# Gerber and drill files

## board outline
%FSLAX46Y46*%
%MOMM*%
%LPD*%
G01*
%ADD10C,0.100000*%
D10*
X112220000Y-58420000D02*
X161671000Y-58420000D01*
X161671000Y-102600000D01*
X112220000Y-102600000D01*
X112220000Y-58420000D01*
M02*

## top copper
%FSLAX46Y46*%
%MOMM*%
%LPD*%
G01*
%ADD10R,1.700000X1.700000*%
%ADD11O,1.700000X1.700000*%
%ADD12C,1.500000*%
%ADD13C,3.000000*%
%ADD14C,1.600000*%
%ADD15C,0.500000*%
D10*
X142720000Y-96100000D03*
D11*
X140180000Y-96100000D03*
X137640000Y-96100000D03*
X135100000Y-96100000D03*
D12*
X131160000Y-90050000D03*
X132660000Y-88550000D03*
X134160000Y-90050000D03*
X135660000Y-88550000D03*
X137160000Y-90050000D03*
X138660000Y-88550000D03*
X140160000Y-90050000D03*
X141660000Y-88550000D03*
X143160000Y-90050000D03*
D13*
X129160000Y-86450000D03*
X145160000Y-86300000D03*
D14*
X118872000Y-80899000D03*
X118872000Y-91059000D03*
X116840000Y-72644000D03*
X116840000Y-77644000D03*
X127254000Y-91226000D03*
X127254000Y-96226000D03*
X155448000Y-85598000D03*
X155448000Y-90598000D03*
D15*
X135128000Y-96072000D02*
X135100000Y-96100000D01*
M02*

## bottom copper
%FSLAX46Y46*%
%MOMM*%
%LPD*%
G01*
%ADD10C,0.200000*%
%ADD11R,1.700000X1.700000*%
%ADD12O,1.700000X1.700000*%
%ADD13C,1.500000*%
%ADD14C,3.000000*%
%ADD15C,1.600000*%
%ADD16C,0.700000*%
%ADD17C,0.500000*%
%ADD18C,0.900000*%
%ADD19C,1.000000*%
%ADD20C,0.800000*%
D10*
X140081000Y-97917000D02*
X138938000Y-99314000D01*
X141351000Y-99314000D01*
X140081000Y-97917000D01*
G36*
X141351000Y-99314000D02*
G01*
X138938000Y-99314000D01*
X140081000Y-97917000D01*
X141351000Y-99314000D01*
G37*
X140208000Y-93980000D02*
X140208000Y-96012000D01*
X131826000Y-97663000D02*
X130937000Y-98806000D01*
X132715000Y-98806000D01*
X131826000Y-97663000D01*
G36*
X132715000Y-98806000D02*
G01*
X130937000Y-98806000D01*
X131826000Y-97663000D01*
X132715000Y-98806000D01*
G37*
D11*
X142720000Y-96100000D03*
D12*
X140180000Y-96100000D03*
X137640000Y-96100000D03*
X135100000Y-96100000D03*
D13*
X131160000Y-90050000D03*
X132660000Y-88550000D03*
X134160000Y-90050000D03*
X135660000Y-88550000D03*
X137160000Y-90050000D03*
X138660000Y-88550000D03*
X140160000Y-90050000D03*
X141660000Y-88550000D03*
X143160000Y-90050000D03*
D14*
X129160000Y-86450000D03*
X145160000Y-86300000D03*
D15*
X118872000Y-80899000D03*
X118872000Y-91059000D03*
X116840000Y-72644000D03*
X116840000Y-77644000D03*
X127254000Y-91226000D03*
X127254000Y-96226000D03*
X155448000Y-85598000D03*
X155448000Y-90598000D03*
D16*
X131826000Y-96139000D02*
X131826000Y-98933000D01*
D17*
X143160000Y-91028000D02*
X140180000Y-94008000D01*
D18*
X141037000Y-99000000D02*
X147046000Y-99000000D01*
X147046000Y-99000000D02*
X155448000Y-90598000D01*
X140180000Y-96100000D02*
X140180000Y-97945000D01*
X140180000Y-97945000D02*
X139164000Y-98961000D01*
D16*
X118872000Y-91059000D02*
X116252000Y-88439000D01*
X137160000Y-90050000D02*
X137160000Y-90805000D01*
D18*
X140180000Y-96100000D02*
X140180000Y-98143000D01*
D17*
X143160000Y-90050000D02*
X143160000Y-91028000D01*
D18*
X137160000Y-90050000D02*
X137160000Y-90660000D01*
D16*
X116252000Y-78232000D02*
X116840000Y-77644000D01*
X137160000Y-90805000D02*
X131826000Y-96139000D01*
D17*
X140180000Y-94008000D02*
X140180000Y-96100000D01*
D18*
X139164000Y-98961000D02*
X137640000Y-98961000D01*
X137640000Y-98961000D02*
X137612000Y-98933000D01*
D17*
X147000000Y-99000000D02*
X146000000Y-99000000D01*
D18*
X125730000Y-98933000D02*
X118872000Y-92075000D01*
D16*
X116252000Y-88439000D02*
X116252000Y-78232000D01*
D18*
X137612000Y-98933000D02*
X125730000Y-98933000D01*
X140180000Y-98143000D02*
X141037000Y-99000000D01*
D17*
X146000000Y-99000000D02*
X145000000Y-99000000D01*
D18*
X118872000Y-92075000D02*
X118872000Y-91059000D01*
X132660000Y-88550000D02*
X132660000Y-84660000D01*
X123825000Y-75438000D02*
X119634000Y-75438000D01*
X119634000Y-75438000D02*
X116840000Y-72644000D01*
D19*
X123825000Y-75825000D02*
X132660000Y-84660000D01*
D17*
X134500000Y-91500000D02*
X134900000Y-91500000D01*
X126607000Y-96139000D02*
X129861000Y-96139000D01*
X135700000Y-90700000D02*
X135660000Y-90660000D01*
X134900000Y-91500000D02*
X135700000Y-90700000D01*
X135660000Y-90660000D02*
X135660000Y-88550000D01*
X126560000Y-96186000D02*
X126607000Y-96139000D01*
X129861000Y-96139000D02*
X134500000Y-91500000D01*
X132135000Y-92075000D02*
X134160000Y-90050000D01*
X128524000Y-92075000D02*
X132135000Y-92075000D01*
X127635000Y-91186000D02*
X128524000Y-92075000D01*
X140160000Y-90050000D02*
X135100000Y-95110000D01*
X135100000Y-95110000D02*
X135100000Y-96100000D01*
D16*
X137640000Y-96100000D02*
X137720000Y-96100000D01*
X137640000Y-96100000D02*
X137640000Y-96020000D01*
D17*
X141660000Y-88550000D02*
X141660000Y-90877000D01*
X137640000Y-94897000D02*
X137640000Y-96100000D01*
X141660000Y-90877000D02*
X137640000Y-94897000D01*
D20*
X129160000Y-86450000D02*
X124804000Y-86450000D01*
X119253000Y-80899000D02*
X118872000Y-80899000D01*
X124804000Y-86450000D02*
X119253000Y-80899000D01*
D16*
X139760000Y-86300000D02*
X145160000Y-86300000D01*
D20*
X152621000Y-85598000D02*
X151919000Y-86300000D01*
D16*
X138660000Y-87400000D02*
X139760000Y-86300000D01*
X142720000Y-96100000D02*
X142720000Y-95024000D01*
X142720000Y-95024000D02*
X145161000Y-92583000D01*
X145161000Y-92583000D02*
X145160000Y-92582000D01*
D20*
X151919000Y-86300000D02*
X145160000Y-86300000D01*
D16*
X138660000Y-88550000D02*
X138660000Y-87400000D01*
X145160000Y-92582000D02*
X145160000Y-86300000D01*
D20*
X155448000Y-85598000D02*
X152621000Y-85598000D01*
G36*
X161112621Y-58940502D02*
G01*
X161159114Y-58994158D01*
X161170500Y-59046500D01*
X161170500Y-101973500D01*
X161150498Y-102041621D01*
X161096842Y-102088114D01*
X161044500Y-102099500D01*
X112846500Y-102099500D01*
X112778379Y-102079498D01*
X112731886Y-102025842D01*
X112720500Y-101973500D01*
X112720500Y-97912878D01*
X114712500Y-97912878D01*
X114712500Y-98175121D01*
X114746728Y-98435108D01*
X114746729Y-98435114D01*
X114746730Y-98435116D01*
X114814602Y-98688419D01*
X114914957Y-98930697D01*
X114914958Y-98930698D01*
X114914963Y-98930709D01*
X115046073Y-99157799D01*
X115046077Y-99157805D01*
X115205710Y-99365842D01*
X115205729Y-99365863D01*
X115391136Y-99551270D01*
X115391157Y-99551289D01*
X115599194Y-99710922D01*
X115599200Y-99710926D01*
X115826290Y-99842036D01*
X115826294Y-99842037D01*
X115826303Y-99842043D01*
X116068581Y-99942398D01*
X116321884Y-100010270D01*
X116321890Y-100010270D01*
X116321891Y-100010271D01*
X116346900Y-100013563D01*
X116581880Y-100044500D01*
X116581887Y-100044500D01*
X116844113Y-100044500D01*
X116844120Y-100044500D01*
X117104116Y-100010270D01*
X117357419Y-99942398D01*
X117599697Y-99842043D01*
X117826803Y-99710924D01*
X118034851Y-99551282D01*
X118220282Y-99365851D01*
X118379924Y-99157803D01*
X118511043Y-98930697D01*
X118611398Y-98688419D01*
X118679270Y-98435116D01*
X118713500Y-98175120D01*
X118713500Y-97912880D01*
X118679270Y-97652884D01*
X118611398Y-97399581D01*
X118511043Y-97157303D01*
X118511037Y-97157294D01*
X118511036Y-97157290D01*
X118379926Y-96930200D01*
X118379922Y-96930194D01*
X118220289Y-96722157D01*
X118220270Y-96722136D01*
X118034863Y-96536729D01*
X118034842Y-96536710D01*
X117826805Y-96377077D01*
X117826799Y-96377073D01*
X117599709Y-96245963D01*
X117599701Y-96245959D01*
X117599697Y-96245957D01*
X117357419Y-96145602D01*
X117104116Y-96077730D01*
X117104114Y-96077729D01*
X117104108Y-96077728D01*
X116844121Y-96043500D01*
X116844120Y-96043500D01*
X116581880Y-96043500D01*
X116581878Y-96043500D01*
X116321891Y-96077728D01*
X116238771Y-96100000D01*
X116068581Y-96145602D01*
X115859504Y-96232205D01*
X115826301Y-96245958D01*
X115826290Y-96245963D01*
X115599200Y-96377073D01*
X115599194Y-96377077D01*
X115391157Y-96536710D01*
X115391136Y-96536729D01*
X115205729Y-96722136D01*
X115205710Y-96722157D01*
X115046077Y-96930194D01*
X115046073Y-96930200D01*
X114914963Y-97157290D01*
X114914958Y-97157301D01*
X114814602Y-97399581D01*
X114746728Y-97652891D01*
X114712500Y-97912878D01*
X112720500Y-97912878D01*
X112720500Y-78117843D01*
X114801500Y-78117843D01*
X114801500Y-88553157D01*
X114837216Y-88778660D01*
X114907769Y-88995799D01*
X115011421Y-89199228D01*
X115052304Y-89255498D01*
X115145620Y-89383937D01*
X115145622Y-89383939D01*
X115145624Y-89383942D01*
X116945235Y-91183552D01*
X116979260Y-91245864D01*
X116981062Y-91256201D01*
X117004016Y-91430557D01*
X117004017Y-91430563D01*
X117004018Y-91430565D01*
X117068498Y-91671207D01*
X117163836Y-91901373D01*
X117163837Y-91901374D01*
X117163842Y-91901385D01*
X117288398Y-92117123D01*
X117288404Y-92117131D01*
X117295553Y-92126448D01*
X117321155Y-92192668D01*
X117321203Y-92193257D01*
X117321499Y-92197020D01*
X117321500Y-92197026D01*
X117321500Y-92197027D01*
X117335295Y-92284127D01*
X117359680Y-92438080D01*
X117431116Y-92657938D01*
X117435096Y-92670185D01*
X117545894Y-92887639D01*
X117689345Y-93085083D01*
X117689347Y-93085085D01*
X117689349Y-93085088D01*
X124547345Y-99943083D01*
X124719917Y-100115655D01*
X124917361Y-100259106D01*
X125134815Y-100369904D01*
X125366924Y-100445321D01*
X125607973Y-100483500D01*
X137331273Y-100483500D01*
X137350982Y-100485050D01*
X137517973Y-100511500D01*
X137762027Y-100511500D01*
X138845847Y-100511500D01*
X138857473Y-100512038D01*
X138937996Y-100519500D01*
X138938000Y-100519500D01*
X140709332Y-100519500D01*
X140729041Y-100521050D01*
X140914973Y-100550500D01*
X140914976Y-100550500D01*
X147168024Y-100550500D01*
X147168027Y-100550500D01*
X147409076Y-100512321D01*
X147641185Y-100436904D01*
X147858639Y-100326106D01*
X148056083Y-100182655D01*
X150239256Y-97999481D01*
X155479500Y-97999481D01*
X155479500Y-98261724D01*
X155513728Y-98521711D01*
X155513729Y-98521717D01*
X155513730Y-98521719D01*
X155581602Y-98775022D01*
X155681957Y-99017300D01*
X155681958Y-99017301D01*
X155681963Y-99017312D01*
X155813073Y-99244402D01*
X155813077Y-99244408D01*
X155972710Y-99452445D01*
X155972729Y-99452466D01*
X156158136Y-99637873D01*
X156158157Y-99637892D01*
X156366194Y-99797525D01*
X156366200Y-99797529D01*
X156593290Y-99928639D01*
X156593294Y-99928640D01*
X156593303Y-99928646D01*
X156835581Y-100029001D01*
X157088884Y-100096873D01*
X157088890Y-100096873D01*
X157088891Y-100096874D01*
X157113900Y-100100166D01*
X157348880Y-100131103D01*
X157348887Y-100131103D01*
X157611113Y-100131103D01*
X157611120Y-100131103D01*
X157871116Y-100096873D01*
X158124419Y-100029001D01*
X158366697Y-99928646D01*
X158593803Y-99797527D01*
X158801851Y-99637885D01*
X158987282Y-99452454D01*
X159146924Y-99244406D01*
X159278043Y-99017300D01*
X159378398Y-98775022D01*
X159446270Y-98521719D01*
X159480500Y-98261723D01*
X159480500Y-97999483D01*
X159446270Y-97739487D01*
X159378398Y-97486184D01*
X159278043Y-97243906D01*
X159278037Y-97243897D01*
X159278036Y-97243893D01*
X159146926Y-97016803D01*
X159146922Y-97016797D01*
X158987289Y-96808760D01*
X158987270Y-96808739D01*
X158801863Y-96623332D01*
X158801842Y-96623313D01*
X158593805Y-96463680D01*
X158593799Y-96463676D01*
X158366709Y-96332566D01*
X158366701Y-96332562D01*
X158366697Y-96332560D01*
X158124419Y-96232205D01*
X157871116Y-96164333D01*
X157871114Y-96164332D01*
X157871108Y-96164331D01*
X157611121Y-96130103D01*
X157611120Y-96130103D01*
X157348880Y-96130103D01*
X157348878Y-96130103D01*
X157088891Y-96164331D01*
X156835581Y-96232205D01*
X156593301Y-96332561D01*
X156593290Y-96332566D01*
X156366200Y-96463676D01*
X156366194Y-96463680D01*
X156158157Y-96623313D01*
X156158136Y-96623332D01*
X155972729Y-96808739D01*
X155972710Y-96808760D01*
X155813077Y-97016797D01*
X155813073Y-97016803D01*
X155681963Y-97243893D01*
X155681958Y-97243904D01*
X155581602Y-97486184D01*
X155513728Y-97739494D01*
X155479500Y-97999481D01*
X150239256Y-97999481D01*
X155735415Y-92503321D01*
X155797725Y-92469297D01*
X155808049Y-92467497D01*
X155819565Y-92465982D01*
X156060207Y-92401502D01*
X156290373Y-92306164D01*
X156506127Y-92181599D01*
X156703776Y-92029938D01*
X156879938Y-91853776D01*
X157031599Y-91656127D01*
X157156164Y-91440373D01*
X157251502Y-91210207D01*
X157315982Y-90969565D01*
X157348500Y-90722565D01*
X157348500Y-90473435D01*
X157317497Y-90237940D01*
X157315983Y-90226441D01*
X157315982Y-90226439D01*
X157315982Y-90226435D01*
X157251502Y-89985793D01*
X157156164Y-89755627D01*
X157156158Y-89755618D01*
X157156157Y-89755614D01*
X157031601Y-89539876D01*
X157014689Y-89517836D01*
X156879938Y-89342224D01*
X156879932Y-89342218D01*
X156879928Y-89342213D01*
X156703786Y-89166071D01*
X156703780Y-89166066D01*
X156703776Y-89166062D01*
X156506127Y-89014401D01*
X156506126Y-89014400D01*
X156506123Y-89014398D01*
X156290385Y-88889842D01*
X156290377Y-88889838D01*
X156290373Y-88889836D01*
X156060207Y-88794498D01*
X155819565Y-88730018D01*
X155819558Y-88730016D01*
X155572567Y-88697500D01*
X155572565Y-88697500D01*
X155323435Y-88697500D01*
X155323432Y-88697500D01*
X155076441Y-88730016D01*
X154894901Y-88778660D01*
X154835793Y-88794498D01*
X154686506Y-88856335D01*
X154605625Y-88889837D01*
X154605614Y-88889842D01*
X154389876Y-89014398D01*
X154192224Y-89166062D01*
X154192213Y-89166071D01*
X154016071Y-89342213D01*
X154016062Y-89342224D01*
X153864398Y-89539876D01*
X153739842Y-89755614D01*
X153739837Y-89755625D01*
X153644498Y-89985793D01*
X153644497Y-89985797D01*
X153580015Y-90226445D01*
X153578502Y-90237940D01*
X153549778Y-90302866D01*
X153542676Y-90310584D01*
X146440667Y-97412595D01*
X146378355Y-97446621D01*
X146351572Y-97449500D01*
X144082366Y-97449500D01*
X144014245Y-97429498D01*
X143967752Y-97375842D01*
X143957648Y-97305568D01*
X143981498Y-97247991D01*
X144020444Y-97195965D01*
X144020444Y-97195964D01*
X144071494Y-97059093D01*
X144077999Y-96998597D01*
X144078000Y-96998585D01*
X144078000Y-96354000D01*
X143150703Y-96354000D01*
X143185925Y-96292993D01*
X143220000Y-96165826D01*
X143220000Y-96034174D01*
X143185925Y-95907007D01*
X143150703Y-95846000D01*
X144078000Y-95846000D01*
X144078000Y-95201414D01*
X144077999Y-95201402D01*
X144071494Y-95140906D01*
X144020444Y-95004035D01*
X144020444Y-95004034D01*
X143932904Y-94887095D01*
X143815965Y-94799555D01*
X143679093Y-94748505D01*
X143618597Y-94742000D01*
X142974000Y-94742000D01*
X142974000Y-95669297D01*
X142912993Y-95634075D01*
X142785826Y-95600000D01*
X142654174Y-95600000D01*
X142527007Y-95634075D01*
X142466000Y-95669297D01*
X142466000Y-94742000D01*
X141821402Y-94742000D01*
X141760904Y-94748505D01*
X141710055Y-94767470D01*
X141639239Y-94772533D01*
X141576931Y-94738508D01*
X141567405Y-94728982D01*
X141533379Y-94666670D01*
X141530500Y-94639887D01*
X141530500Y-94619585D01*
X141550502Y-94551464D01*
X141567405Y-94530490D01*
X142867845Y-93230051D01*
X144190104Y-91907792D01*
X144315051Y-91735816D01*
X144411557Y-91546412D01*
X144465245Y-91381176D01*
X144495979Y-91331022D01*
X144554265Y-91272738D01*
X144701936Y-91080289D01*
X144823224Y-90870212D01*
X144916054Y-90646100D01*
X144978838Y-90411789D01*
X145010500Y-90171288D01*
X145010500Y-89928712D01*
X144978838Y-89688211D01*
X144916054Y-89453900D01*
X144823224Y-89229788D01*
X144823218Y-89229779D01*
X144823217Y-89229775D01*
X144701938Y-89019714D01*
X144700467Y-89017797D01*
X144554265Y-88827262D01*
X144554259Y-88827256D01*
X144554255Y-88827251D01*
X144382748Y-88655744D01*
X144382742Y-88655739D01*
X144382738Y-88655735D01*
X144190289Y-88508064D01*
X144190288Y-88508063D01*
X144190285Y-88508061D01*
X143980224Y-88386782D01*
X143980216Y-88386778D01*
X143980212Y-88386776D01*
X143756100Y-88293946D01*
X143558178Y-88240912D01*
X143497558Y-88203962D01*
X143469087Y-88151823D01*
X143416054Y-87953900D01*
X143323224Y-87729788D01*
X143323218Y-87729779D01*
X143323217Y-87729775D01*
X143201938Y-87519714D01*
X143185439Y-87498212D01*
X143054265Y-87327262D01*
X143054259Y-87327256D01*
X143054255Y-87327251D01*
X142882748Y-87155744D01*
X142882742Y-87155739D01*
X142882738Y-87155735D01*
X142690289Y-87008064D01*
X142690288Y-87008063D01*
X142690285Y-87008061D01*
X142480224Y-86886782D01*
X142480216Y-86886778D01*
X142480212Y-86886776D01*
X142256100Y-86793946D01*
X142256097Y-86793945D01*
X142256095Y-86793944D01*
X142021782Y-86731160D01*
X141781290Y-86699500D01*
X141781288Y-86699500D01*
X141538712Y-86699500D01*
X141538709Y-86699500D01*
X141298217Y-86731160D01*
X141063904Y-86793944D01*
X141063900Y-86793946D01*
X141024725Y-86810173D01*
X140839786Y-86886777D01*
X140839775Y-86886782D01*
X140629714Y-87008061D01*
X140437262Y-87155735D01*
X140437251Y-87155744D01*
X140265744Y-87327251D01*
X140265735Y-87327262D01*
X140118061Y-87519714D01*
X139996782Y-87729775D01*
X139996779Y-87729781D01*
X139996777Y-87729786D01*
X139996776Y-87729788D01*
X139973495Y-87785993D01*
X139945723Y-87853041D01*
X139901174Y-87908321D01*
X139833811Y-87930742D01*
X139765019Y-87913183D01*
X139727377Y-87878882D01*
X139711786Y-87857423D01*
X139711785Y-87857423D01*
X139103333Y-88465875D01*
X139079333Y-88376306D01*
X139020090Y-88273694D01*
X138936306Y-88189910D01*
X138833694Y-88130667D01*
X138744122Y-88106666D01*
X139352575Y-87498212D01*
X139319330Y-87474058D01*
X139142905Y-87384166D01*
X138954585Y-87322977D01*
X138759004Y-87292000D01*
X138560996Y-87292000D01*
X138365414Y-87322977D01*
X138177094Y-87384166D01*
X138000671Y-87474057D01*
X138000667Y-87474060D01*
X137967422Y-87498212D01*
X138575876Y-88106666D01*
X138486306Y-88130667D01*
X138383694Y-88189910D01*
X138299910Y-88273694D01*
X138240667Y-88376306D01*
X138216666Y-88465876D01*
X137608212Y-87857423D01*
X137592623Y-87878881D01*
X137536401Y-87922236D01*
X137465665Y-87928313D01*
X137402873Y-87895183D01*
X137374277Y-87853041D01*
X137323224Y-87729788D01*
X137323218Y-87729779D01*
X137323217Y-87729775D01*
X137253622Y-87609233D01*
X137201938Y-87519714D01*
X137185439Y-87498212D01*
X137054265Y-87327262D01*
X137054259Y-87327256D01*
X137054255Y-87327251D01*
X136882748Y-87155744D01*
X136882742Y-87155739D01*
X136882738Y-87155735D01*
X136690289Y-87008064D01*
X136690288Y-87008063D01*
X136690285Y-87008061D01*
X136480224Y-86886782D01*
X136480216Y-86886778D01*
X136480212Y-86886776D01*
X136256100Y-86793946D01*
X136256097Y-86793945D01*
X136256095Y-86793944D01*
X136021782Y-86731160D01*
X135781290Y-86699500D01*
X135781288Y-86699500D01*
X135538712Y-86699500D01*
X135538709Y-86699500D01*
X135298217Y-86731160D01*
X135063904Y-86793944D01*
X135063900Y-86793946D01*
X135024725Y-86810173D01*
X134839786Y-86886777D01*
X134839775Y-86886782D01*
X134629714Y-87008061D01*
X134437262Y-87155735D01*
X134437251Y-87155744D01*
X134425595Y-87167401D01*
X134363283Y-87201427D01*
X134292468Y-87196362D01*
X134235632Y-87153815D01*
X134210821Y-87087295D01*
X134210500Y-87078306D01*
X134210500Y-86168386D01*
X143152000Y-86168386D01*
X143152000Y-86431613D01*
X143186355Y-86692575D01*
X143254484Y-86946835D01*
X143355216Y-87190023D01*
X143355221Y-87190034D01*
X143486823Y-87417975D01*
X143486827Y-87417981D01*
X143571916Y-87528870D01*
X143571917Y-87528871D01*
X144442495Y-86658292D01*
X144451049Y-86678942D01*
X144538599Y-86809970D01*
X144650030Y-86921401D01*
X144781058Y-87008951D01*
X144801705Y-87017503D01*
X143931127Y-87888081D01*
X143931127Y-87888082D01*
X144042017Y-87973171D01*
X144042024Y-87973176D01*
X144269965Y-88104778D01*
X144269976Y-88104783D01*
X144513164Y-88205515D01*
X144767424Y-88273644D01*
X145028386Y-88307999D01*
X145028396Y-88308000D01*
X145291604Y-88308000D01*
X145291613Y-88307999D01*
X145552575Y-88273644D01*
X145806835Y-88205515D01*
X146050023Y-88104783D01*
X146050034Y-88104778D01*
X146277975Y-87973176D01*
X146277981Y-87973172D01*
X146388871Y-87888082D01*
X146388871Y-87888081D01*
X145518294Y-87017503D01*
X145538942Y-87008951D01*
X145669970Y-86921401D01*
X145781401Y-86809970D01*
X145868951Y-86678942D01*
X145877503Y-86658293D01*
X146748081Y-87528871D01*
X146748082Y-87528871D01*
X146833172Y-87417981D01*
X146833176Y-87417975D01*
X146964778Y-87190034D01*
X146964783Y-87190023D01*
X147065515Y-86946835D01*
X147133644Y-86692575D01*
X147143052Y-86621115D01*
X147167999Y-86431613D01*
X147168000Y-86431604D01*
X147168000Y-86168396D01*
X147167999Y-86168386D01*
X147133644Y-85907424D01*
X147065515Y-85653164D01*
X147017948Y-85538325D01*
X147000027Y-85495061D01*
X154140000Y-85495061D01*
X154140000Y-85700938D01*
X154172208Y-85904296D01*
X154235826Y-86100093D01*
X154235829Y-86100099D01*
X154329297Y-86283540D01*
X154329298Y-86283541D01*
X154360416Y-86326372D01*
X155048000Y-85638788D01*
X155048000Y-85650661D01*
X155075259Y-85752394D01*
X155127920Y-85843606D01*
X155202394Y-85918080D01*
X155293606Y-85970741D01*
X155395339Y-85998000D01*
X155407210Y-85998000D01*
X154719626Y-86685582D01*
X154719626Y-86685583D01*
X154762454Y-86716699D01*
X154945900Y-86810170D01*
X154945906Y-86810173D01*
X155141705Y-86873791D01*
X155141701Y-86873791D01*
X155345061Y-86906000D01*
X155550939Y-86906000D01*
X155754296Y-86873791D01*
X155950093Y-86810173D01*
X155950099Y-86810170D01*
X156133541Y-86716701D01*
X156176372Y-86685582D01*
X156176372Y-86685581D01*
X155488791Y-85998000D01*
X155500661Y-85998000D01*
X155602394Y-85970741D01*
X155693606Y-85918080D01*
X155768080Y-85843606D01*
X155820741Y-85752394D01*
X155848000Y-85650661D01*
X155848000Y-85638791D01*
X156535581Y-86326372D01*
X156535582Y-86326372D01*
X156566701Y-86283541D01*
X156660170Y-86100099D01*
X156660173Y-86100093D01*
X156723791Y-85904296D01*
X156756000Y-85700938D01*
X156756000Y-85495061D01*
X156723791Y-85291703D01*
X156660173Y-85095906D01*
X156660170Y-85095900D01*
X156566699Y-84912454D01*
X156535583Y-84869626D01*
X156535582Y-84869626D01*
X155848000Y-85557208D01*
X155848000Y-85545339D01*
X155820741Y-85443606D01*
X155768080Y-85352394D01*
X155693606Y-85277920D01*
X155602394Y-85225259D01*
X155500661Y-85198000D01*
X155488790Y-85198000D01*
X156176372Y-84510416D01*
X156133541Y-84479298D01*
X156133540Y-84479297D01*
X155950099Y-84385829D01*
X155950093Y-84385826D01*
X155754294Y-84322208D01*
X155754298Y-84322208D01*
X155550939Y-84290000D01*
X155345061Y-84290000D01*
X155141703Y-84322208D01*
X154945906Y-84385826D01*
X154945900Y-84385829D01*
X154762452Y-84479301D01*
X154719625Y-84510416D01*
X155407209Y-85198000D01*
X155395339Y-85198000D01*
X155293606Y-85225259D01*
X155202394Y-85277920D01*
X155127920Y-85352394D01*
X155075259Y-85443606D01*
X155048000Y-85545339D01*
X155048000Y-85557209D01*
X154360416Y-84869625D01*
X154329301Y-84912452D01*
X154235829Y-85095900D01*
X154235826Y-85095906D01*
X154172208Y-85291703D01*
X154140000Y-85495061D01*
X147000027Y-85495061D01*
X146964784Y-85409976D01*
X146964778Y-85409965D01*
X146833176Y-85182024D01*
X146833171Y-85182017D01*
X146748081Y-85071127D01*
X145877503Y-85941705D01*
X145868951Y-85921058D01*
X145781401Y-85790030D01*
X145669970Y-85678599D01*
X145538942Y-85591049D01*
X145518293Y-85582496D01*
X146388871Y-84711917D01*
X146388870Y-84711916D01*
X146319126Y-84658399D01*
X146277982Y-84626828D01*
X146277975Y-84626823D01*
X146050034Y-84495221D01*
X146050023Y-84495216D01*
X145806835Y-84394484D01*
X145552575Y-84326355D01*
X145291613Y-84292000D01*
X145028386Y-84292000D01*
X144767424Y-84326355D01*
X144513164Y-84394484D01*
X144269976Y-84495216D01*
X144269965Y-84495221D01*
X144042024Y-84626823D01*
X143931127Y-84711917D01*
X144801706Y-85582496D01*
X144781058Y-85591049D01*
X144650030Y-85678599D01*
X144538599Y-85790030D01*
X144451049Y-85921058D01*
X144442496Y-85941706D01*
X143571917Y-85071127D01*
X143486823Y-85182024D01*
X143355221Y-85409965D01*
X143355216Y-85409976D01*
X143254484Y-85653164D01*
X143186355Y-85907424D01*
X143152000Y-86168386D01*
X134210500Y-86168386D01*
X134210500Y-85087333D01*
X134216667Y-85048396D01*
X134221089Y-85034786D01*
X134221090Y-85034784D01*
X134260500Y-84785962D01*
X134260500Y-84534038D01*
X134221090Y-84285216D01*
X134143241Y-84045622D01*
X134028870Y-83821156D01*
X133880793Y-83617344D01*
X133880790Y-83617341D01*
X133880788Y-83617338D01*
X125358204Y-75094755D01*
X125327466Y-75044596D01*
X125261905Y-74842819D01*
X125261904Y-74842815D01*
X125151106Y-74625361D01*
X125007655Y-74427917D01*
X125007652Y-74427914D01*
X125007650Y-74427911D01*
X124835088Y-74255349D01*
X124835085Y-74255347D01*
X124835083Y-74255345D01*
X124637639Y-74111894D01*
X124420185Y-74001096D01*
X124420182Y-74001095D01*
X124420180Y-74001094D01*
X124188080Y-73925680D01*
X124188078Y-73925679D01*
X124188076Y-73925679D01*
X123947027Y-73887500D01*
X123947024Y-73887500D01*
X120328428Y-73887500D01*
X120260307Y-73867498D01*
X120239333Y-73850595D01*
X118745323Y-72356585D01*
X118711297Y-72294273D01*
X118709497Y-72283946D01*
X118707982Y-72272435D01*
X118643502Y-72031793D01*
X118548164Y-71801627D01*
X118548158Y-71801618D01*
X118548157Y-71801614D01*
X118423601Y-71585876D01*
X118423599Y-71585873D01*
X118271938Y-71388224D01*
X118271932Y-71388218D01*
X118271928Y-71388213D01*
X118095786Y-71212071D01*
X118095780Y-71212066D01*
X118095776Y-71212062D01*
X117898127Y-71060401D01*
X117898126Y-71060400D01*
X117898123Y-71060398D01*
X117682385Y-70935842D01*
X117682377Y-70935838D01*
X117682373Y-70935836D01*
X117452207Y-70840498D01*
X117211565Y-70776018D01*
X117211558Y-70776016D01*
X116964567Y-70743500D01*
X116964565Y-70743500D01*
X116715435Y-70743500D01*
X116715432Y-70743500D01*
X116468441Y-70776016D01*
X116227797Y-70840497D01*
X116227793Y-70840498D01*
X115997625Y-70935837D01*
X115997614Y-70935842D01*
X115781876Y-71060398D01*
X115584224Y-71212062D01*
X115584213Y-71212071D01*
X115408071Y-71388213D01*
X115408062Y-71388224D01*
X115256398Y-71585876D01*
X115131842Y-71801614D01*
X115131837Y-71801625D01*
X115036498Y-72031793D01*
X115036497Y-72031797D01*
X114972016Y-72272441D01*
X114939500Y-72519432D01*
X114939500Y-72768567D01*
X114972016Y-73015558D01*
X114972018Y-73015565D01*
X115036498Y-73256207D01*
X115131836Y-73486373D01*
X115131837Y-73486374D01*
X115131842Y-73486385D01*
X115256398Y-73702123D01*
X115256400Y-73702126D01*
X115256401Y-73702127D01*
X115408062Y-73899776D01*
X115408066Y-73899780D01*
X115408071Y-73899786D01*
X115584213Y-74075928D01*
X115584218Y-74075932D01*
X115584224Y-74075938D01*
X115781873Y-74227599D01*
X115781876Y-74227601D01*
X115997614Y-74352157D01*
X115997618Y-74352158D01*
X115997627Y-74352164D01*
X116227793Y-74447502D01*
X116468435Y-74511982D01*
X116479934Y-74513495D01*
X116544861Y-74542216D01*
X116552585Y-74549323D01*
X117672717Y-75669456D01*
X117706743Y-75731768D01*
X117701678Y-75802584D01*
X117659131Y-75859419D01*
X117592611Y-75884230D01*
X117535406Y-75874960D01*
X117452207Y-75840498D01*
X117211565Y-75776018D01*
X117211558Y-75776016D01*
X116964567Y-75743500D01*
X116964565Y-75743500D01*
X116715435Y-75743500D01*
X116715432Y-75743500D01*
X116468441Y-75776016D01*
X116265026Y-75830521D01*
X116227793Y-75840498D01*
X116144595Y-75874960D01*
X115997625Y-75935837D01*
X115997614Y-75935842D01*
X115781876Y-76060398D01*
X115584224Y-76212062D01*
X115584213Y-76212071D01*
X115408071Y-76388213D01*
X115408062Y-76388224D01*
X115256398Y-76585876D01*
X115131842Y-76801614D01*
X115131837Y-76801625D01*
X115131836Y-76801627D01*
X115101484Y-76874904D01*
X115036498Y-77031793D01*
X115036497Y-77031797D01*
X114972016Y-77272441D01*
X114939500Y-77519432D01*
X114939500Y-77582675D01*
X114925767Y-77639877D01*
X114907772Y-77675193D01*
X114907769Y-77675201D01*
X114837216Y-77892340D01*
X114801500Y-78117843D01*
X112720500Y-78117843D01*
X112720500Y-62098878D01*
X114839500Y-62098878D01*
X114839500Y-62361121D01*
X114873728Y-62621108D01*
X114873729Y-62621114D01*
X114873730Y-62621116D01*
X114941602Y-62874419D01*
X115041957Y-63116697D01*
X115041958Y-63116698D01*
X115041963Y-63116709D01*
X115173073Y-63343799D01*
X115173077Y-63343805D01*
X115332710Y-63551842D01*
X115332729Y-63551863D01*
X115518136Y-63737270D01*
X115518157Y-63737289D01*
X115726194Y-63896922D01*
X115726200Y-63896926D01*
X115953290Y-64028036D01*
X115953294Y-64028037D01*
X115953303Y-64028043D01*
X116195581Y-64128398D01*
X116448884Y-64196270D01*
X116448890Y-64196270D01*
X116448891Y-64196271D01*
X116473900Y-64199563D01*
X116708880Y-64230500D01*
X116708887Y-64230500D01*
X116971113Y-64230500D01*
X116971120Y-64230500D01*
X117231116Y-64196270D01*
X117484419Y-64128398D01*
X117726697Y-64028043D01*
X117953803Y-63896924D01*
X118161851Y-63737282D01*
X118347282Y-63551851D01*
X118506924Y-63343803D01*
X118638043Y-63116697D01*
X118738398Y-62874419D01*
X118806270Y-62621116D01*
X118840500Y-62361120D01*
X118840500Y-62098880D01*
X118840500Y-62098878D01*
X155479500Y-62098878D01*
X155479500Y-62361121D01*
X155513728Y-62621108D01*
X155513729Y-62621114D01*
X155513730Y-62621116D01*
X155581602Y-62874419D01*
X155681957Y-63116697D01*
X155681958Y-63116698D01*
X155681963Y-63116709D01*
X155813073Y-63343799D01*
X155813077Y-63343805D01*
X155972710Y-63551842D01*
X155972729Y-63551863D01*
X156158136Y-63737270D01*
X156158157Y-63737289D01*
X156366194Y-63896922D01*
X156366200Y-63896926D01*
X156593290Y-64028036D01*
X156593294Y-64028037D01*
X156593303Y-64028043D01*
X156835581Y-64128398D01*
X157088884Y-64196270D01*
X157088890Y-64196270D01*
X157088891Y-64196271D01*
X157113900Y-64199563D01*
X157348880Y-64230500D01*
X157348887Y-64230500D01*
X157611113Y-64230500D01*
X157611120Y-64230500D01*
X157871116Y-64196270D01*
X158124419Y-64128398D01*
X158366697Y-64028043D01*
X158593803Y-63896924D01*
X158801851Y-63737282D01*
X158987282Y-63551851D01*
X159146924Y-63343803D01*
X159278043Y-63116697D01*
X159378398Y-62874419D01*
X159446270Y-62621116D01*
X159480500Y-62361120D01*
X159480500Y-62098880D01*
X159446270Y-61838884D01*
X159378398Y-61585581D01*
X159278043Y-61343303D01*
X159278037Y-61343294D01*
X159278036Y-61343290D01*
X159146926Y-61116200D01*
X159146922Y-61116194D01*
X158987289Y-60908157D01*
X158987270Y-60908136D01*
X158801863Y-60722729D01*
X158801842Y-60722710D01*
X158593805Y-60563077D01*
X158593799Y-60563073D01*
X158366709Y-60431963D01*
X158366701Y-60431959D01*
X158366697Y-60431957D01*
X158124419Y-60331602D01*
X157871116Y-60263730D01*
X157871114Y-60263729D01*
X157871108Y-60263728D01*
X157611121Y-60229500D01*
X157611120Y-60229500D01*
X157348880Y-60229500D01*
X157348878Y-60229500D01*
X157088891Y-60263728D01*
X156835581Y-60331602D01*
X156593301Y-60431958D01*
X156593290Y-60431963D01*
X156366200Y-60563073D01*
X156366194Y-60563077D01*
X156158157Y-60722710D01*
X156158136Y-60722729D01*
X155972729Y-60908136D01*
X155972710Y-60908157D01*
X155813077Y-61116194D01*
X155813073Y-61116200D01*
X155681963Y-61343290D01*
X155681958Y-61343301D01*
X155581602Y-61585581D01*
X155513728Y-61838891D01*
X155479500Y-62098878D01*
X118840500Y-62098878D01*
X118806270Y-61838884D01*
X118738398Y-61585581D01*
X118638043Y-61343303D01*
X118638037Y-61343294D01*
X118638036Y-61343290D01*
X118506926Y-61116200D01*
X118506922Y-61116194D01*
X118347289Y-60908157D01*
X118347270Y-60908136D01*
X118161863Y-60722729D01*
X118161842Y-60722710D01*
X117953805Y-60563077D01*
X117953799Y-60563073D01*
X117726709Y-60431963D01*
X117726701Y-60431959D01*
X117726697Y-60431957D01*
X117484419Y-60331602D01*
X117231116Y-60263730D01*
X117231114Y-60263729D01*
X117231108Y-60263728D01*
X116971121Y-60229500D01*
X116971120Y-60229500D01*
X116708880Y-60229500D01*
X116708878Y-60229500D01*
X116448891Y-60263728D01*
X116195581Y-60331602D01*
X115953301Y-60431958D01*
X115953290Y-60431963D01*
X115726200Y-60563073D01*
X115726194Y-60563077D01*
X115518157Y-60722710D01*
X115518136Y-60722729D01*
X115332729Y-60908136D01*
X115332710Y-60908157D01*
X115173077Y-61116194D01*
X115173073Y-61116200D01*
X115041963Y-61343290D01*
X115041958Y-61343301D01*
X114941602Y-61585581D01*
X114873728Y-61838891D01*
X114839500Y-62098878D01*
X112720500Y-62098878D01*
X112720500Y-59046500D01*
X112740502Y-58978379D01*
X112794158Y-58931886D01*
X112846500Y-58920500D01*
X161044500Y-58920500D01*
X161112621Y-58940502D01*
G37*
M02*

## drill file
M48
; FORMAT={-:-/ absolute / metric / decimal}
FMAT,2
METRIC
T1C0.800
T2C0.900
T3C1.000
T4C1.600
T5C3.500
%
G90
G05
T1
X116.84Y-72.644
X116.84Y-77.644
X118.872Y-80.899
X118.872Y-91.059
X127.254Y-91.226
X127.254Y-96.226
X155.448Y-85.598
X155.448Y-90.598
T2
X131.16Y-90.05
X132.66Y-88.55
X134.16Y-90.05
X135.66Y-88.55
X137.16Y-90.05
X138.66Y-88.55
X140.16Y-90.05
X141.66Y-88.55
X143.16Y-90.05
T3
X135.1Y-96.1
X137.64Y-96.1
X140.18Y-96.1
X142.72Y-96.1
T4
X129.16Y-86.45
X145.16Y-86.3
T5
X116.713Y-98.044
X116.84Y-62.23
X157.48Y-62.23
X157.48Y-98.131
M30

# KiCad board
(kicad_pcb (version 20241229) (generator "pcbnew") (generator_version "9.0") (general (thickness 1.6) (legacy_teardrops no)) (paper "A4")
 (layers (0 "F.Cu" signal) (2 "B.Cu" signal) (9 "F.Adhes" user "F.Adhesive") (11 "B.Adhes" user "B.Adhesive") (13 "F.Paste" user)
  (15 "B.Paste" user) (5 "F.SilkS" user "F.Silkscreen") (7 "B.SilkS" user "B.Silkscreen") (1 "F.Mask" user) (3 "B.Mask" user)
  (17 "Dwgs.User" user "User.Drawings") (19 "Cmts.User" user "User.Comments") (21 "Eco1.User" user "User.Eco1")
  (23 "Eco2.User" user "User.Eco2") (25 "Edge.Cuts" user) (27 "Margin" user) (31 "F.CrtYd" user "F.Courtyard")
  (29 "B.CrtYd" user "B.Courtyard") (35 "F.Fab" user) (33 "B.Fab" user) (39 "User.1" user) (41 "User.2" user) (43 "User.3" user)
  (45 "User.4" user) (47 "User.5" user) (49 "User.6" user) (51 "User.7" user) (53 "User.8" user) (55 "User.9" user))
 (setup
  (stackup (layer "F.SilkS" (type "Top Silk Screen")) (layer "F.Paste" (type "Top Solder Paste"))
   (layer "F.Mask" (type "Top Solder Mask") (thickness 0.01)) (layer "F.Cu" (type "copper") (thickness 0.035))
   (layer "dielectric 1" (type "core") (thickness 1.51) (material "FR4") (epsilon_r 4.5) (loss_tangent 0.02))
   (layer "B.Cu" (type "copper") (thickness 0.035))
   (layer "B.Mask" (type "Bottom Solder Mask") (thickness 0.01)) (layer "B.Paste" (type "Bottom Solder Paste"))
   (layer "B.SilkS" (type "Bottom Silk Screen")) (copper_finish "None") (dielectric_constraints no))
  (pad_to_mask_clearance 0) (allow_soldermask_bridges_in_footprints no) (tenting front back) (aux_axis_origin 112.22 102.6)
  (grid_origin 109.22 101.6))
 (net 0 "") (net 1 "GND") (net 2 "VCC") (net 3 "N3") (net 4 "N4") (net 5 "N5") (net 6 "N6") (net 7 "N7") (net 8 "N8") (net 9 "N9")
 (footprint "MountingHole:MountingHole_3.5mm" (layer "F.Cu") (at 157.48 62.23)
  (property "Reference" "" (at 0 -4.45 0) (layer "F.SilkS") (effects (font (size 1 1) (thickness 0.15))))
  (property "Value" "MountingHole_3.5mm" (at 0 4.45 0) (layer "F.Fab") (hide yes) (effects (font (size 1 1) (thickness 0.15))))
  (pad "" np_thru_hole circle (at 0 0) (size 3.5 3.5) (drill 3.5) (layers "*.Cu" "*.Mask")))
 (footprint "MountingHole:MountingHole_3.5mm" (layer "F.Cu") (at 157.48 98.130603)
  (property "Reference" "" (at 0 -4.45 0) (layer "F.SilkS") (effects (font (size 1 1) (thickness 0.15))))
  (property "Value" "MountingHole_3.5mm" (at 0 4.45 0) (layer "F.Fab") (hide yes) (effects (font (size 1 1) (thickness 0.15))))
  (pad "" np_thru_hole circle (at 0 0) (size 3.5 3.5) (drill 3.5) (layers "*.Cu" "*.Mask")))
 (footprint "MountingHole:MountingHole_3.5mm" (layer "F.Cu") (at 116.84 62.23)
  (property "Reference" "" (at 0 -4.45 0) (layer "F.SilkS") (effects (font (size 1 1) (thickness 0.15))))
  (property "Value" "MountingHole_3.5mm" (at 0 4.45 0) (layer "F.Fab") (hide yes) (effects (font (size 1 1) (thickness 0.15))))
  (pad "" np_thru_hole circle (at 0 0) (size 3.5 3.5) (drill 3.5) (layers "*.Cu" "*.Mask")))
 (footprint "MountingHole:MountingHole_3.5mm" (layer "F.Cu") (at 116.713 98.044)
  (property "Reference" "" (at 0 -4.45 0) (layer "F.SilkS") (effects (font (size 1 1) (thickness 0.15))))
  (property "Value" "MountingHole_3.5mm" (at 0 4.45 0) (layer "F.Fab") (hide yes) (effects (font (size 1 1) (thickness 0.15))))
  (pad "" np_thru_hole circle (at 0 0) (size 3.5 3.5) (drill 3.5) (layers "*.Cu" "*.Mask")))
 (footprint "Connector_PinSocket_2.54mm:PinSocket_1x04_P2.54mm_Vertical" (layer "F.Cu") (at 142.72 96.1 -90)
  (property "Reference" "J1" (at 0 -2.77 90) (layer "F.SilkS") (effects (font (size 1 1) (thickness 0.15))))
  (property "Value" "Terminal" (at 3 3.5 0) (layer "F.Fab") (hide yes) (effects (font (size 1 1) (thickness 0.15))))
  (pad "1" thru_hole rect (at 0 0 270) (size 1.7 1.7) (drill 1) (layers "*.Cu" "*.Mask") (remove_unused_layers no) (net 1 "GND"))
  (pad "2" thru_hole oval (at 0 2.54 270) (size 1.7 1.7) (drill 1) (layers "*.Cu" "*.Mask") (remove_unused_layers no) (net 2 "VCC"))
  (pad "3" thru_hole oval (at 0 5.08 270) (size 1.7 1.7) (drill 1) (layers "*.Cu" "*.Mask") (remove_unused_layers no) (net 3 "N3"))
  (pad "4" thru_hole oval (at 0 7.62 270) (size 1.7 1.7) (drill 1) (layers "*.Cu" "*.Mask") (remove_unused_layers no) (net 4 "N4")))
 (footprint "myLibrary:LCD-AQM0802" (layer "F.Cu") (at 137.16 88.55)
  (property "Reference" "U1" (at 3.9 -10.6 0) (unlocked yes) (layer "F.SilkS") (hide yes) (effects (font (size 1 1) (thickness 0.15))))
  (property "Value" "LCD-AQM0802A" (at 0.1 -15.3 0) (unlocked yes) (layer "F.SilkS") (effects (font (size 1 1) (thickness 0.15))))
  (pad "1" thru_hole circle (at -6 1.5) (size 1.5 1.5) (drill 0.9) (layers "*.Cu" "*.Mask") (remove_unused_layers no) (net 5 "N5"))
  (pad "2" thru_hole circle (at -4.5 0) (size 1.5 1.5) (drill 0.9) (layers "*.Cu" "*.Mask") (remove_unused_layers no) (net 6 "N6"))
  (pad "3" thru_hole circle (at -3 1.5) (size 1.5 1.5) (drill 0.9) (layers "*.Cu" "*.Mask") (remove_unused_layers no) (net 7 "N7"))
  (pad "4" thru_hole circle (at -1.5 0) (size 1.5 1.5) (drill 0.9) (layers "*.Cu" "*.Mask") (remove_unused_layers no) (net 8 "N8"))
  (pad "5" thru_hole circle (at 0 1.5) (size 1.5 1.5) (drill 0.9) (layers "*.Cu" "*.Mask") (remove_unused_layers no) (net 2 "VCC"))
  (pad "6" thru_hole circle (at 1.5 0) (size 1.5 1.5) (drill 0.9) (layers "*.Cu" "*.Mask") (remove_unused_layers no) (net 1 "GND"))
  (pad "7" thru_hole circle (at 3 1.5) (size 1.5 1.5) (drill 0.9) (layers "*.Cu" "*.Mask") (remove_unused_layers no) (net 4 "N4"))
  (pad "8" thru_hole circle (at 4.5 0) (size 1.5 1.5) (drill 0.9) (layers "*.Cu" "*.Mask") (remove_unused_layers no) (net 3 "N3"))
  (pad "9" thru_hole circle (at 6 1.5) (size 1.5 1.5) (drill 0.9) (layers "*.Cu" "*.Mask") (remove_unused_layers yes) (keep_end_layers yes)
   (zone_layer_connections) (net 2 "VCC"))
  (pad "10" thru_hole circle (at -8 -2.1 90) (size 3 3) (drill 1.6) (layers "*.Cu" "*.Mask") (remove_unused_layers yes)
   (keep_end_layers yes) (zone_layer_connections) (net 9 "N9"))
  (pad "11" thru_hole circle (at 8 -2.25 90) (size 3 3) (drill 1.6) (layers "*.Cu" "*.Mask") (remove_unused_layers no) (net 1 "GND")))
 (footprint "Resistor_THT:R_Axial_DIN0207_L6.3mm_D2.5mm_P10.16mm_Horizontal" (layer "B.Cu") (at 118.872 80.899 -90)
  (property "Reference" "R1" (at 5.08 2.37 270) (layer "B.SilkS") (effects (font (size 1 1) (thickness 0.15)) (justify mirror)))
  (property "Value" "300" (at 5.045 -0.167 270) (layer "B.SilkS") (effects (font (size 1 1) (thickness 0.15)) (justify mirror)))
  (pad "1" thru_hole circle (at 0 0 270) (size 1.6 1.6) (drill 0.8) (layers "*.Cu" "*.Mask") (remove_unused_layers no) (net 9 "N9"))
  (pad "2" thru_hole circle (at 10.16 0 270) (size 1.6 1.6) (drill 0.8) (layers "*.Cu" "*.Mask") (remove_unused_layers no) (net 2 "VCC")))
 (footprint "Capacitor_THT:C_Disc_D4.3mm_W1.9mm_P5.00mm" (layer "B.Cu") (at 116.84 72.644 -90)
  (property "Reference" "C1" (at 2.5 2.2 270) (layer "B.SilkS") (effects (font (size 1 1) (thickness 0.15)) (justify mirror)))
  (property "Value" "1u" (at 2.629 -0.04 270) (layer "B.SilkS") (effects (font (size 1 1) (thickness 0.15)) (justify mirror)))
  (pad "1" thru_hole circle (at 0 0 270) (size 1.6 1.6) (drill 0.8) (layers "*.Cu" "*.Mask") (remove_unused_layers no) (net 6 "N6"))
  (pad "2" thru_hole circle (at 5 0 270) (size 1.6 1.6) (drill 0.8) (layers "*.Cu" "*.Mask") (remove_unused_layers no) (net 2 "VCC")))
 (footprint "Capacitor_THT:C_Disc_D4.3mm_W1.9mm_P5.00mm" (layer "B.Cu") (at 127.254 91.226 -90)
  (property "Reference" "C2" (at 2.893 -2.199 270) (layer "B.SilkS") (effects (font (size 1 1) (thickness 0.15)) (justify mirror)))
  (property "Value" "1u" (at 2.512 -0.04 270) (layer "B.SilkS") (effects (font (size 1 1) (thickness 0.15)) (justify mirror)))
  (pad "1" thru_hole circle (at 0 0 270) (size 1.6 1.6) (drill 0.8) (layers "*.Cu" "*.Mask") (remove_unused_layers no) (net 7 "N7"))
  (pad "2" thru_hole circle (at 5 0 270) (size 1.6 1.6) (drill 0.8) (layers "*.Cu" "*.Mask") (remove_unused_layers no) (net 8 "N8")))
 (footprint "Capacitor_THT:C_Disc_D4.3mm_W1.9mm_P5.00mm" (layer "B.Cu") (at 155.448 85.598 -90)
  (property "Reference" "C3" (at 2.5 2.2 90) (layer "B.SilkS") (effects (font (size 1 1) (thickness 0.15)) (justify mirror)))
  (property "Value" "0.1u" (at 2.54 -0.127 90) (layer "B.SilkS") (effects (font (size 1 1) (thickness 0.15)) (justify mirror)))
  (pad "1" thru_hole circle (at 0 0 270) (size 1.6 1.6) (drill 0.8) (layers "*.Cu" "*.Mask") (remove_unused_layers no) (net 1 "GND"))
  (pad "2" thru_hole circle (at 5 0 270) (size 1.6 1.6) (drill 0.8) (layers "*.Cu" "*.Mask") (remove_unused_layers no) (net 2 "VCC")))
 (gr_poly
  (pts (xy 140.081 97.917) (xy 138.938 99.314) (xy 141.351 99.314)) (stroke (width 0.2) (type solid)) (fill yes) (layer "B.Cu") (net 2))
 (gr_line (start 140.208 93.98) (end 140.208 96.012) (stroke (width 0.2) (type default)) (layer "B.Cu") (net 2))
 (gr_poly
  (pts (xy 131.826 97.663) (xy 130.937 98.806) (xy 132.715 98.806)) (stroke (width 0.2) (type solid)) (fill yes) (layer "B.Cu") (net 2))
 (gr_rect (start 112.22 58.42) (end 161.671 102.6) (stroke (width 0.1) (type solid)) (fill no) (layer "Edge.Cuts"))
 (segment (start 131.826 96.139) (end 131.826 98.933) (width 0.7) (layer "B.Cu") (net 2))
 (segment (start 143.16 91.028) (end 140.18 94.008) (width 0.5) (layer "B.Cu") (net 2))
 (segment (start 141.037 99) (end 147.046 99) (width 0.9) (layer "B.Cu") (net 2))
 (segment (start 147.046 99) (end 155.448 90.598) (width 0.9) (layer "B.Cu") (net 2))
 (segment (start 140.18 96.1) (end 140.18 97.945) (width 0.9) (layer "B.Cu") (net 2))
 (segment (start 140.18 97.945) (end 139.164 98.961) (width 0.9) (layer "B.Cu") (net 2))
 (segment (start 118.872 91.059) (end 116.252 88.439) (width 0.7) (layer "B.Cu") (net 2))
 (segment (start 137.16 90.05) (end 137.16 90.805) (width 0.7) (layer "B.Cu") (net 2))
 (segment (start 140.18 96.1) (end 140.18 98.143) (width 0.9) (layer "B.Cu") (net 2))
 (segment (start 143.16 90.05) (end 143.16 91.028) (width 0.5) (layer "B.Cu") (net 2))
 (segment (start 137.16 90.05) (end 137.16 90.66) (width 0.9) (layer "B.Cu") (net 2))
 (segment (start 116.252 78.232) (end 116.84 77.644) (width 0.7) (layer "B.Cu") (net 2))
 (segment (start 137.16 90.805) (end 131.826 96.139) (width 0.7) (layer "B.Cu") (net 2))
 (segment (start 140.18 94.008) (end 140.18 96.1) (width 0.5) (layer "B.Cu") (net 2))
 (segment (start 139.164 98.961) (end 137.64 98.961) (width 0.9) (layer "B.Cu") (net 2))
 (segment (start 137.64 98.961) (end 137.612 98.933) (width 0.9) (layer "B.Cu") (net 2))
 (segment (start 147 99) (end 146 99) (width 0.5) (layer "B.Cu") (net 2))
 (segment (start 125.73 98.933) (end 118.872 92.075) (width 0.9) (layer "B.Cu") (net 2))
 (segment (start 116.252 88.439) (end 116.252 78.232) (width 0.7) (layer "B.Cu") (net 2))
 (segment (start 137.612 98.933) (end 125.73 98.933) (width 0.9) (layer "B.Cu") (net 2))
 (segment (start 140.18 98.143) (end 141.037 99) (width 0.9) (layer "B.Cu") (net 2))
 (segment (start 146 99) (end 145 99) (width 0.5) (layer "B.Cu") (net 2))
 (segment (start 118.872 92.075) (end 118.872 91.059) (width 0.9) (layer "B.Cu") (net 2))
 (segment (start 132.66 88.55) (end 132.66 84.66) (width 0.9) (layer "B.Cu") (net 6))
 (segment (start 123.825 75.438) (end 119.634 75.438) (width 0.9) (layer "B.Cu") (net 6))
 (segment (start 119.634 75.438) (end 116.84 72.644) (width 0.9) (layer "B.Cu") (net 6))
 (segment (start 123.825 75.825) (end 132.66 84.66) (width 1) (layer "B.Cu") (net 6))
 (segment (start 134.5 91.5) (end 134.9 91.5) (width 0.5) (layer "B.Cu") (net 8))
 (segment (start 126.607 96.139) (end 129.861 96.139) (width 0.5) (layer "B.Cu") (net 8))
 (segment (start 135.7 90.7) (end 135.66 90.66) (width 0.5) (layer "B.Cu") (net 8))
 (segment (start 134.9 91.5) (end 135.7 90.7) (width 0.5) (layer "B.Cu") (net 8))
 (segment (start 135.66 90.66) (end 135.66 88.55) (width 0.5) (layer "B.Cu") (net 8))
 (segment (start 126.56 96.186) (end 126.607 96.139) (width 0.5) (layer "B.Cu") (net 8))
 (segment (start 129.861 96.139) (end 134.5 91.5) (width 0.5) (layer "B.Cu") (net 8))
 (segment (start 132.135 92.075) (end 134.16 90.05) (width 0.5) (layer "B.Cu") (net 7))
 (segment (start 128.524 92.075) (end 132.135 92.075) (width 0.5) (layer "B.Cu") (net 7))
 (segment (start 127.635 91.186) (end 128.524 92.075) (width 0.5) (layer "B.Cu") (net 7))
 (segment (start 135.128 96.072) (end 135.1 96.1) (width 0.5) (layer "F.Cu") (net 4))
 (segment (start 140.16 90.05) (end 135.1 95.11) (width 0.5) (layer "B.Cu") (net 4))
 (segment (start 135.1 95.11) (end 135.1 96.1) (width 0.5) (layer "B.Cu") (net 4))
 (segment (start 137.64 96.1) (end 137.72 96.1) (width 0.7) (layer "B.Cu") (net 3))
 (segment (start 137.64 96.1) (end 137.64 96.02) (width 0.7) (layer "B.Cu") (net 3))
 (segment (start 141.66 88.55) (end 141.66 90.877) (width 0.5) (layer "B.Cu") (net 3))
 (segment (start 137.64 94.897) (end 137.64 96.1) (width 0.5) (layer "B.Cu") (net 3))
 (segment (start 141.66 90.877) (end 137.64 94.897) (width 0.5) (layer "B.Cu") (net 3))
 (segment (start 129.16 86.45) (end 124.804 86.45) (width 0.8) (layer "B.Cu") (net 9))
 (segment (start 119.253 80.899) (end 118.872 80.899) (width 0.8) (layer "B.Cu") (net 9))
 (segment (start 124.804 86.45) (end 119.253 80.899) (width 0.8) (layer "B.Cu") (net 9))
 (segment (start 139.76 86.3) (end 145.16 86.3) (width 0.7) (layer "B.Cu") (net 1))
 (segment (start 152.621 85.598) (end 151.919 86.3) (width 0.8) (layer "B.Cu") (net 1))
 (segment (start 138.66 87.4) (end 139.76 86.3) (width 0.7) (layer "B.Cu") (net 1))
 (segment (start 142.72 96.1) (end 142.72 95.024) (width 0.7) (layer "B.Cu") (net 1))
 (segment (start 142.72 95.024) (end 145.161 92.583) (width 0.7) (layer "B.Cu") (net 1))
 (segment (start 145.161 92.583) (end 145.16 92.582) (width 0.7) (layer "B.Cu") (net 1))
 (segment (start 151.919 86.3) (end 145.16 86.3) (width 0.8) (layer "B.Cu") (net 1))
 (segment (start 138.66 88.55) (end 138.66 87.4) (width 0.7) (layer "B.Cu") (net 1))
 (segment (start 145.16 92.582) (end 145.16 86.3) (width 0.7) (layer "B.Cu") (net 1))
 (segment (start 155.448 85.598) (end 152.621 85.598) (width 0.8) (layer "B.Cu") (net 1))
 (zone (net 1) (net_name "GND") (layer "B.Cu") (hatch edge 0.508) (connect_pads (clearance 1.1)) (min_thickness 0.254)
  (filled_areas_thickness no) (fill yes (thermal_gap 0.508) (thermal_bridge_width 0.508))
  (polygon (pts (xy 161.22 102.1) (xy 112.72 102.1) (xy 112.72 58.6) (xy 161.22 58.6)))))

